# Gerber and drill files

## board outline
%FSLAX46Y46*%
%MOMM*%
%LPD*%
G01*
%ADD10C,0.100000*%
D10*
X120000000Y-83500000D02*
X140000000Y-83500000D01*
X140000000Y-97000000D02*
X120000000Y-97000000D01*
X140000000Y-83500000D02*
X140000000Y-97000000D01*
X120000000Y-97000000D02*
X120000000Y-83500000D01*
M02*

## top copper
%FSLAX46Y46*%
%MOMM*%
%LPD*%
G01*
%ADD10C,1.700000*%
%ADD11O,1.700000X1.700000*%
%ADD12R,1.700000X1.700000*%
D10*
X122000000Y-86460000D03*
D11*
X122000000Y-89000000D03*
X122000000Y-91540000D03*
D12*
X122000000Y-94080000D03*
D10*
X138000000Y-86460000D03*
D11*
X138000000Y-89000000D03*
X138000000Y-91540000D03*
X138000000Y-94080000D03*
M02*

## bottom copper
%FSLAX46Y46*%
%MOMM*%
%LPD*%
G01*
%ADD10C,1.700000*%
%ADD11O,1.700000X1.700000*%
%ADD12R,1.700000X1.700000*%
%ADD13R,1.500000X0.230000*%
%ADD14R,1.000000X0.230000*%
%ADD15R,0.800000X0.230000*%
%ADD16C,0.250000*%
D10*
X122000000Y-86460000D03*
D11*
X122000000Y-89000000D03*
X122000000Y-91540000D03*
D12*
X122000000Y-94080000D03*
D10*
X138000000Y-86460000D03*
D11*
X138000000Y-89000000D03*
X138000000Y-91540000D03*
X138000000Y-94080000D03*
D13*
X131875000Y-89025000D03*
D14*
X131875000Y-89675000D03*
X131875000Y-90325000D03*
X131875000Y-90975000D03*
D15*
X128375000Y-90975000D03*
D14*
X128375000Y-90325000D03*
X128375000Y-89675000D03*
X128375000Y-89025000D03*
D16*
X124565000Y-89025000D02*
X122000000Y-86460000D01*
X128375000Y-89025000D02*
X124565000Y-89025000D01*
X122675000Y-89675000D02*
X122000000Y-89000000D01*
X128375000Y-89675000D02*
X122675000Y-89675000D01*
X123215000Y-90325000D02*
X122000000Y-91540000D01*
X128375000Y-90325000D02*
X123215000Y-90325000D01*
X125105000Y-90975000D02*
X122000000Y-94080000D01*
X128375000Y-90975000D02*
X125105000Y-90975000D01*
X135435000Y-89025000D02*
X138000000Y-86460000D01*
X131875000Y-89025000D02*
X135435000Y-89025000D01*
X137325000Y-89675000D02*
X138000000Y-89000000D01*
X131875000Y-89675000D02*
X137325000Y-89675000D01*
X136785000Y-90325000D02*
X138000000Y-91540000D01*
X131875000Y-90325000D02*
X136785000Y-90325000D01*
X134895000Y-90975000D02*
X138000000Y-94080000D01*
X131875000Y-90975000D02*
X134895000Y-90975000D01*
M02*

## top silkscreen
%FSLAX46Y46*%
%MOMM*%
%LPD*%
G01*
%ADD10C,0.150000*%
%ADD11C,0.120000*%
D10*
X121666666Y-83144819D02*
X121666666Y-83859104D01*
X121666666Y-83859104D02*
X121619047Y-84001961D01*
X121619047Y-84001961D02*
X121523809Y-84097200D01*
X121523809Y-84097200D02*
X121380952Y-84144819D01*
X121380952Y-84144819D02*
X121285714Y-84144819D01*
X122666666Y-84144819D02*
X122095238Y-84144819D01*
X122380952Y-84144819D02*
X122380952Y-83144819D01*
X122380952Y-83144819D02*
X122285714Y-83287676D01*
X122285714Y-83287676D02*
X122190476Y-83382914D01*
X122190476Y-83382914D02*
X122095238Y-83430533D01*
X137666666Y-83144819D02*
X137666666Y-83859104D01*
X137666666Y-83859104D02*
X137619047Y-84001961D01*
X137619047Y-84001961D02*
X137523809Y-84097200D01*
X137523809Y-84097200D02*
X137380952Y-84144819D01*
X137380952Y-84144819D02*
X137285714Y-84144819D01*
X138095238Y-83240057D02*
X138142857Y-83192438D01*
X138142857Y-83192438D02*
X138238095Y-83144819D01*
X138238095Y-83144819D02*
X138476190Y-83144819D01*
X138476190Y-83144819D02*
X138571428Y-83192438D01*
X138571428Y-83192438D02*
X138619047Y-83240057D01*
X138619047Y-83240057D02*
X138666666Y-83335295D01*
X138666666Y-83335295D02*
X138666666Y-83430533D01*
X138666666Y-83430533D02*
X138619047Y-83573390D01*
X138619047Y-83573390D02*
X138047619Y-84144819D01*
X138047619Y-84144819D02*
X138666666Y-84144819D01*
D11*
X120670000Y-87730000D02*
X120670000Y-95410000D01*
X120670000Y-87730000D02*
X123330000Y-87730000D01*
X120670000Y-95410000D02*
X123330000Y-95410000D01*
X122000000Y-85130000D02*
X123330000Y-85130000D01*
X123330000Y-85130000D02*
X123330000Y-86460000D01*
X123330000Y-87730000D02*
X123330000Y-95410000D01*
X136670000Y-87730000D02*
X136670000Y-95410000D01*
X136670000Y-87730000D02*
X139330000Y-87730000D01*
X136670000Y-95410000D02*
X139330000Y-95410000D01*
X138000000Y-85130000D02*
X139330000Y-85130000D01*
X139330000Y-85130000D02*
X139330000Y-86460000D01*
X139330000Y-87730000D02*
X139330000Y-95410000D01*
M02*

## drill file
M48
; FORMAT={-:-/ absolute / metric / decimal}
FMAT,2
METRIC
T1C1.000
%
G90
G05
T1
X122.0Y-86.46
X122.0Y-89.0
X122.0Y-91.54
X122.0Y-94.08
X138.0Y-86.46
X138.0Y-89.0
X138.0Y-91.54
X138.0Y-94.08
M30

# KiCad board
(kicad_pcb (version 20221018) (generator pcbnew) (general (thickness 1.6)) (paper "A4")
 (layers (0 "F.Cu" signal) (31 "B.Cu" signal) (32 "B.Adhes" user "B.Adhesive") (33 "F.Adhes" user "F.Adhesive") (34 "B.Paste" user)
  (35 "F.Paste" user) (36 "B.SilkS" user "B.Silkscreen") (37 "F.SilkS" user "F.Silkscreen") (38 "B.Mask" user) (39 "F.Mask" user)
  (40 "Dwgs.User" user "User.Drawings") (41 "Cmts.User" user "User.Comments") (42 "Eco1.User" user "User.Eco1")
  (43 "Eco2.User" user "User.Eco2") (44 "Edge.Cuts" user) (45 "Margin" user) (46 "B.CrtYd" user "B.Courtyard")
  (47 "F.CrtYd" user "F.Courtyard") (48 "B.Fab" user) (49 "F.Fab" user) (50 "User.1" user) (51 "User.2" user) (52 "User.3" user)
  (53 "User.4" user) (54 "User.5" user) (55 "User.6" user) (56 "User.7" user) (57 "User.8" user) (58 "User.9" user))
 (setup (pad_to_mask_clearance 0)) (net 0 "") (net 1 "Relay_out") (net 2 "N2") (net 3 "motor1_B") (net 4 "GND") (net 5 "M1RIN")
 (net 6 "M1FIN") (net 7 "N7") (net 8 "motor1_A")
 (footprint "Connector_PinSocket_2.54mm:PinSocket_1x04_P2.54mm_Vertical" (layer "F.Cu") (at 122 86.46)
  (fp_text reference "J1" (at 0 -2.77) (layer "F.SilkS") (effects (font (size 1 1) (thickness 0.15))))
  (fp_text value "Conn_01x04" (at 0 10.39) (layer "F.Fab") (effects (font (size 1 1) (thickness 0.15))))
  (fp_line (start -1.33 1.27) (end -1.33 8.95) (stroke (width 0.12) (type solid)) (layer "F.SilkS"))
  (fp_line (start -1.33 1.27) (end 1.33 1.27) (stroke (width 0.12) (type solid)) (layer "F.SilkS"))
  (fp_line (start -1.33 8.95) (end 1.33 8.95) (stroke (width 0.12) (type solid)) (layer "F.SilkS"))
  (fp_line (start 0 -1.33) (end 1.33 -1.33) (stroke (width 0.12) (type solid)) (layer "F.SilkS"))
  (fp_line (start 1.33 -1.33) (end 1.33 0) (stroke (width 0.12) (type solid)) (layer "F.SilkS"))
  (fp_line (start 1.33 1.27) (end 1.33 8.95) (stroke (width 0.12) (type solid)) (layer "F.SilkS"))
  (pad "1" thru_hole circle (at 0 0) (size 1.7 1.7) (drill 1) (layers "*.Cu" "*.Mask") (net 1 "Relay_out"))
  (pad "2" thru_hole oval (at 0 2.54) (size 1.7 1.7) (drill 1) (layers "*.Cu" "*.Mask") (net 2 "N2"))
  (pad "3" thru_hole oval (at 0 5.08) (size 1.7 1.7) (drill 1) (layers "*.Cu" "*.Mask") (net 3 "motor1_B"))
  (pad "4" thru_hole rect (at 0 7.62) (size 1.7 1.7) (drill 1) (layers "*.Cu" "*.Mask") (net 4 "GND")))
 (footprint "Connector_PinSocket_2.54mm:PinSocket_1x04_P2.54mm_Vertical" (layer "F.Cu") (at 138 86.46)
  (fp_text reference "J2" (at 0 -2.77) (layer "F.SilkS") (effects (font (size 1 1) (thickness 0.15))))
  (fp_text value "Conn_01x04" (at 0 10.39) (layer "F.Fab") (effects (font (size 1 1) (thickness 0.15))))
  (fp_line (start -1.33 1.27) (end -1.33 8.95) (stroke (width 0.12) (type solid)) (layer "F.SilkS"))
  (fp_line (start -1.33 1.27) (end 1.33 1.27) (stroke (width 0.12) (type solid)) (layer "F.SilkS"))
  (fp_line (start -1.33 8.95) (end 1.33 8.95) (stroke (width 0.12) (type solid)) (layer "F.SilkS"))
  (fp_line (start 0 -1.33) (end 1.33 -1.33) (stroke (width 0.12) (type solid)) (layer "F.SilkS"))
  (fp_line (start 1.33 -1.33) (end 1.33 0) (stroke (width 0.12) (type solid)) (layer "F.SilkS"))
  (fp_line (start 1.33 1.27) (end 1.33 8.95) (stroke (width 0.12) (type solid)) (layer "F.SilkS"))
  (pad "1" thru_hole circle (at 0 0) (size 1.7 1.7) (drill 1) (layers "*.Cu" "*.Mask") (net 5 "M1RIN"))
  (pad "2" thru_hole oval (at 0 2.54) (size 1.7 1.7) (drill 1) (layers "*.Cu" "*.Mask") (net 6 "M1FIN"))
  (pad "3" thru_hole oval (at 0 5.08) (size 1.7 1.7) (drill 1) (layers "*.Cu" "*.Mask") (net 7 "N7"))
  (pad "4" thru_hole oval (at 0 7.62) (size 1.7 1.7) (drill 1) (layers "*.Cu" "*.Mask") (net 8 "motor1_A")))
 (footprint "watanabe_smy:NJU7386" (layer "B.Cu") (at 127.875 90 -90)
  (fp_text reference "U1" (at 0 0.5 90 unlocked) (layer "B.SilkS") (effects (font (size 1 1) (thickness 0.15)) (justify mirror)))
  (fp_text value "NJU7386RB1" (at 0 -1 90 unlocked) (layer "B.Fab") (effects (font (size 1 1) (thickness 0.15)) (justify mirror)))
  (pad "1" smd rect (at -0.975 -4 270) (size 0.23 1.5) (layers "B.Cu" "B.Paste" "B.Mask") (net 5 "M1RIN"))
  (pad "2" smd rect (at -0.325 -4 270) (size 0.23 1) (layers "B.Cu" "B.Paste" "B.Mask") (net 6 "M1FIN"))
  (pad "3" smd rect (at 0.325 -4 270) (size 0.23 1) (layers "B.Cu" "B.Paste" "B.Mask") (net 7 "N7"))
  (pad "4" smd rect (at 0.975 -4 270) (size 0.23 1) (layers "B.Cu" "B.Paste" "B.Mask") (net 8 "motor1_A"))
  (pad "5" smd rect (at 0.975 -0.5 270) (size 0.23 0.8) (layers "B.Cu" "B.Paste" "B.Mask") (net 4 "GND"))
  (pad "6" smd rect (at 0.325 -0.5 270) (size 0.23 1) (layers "B.Cu" "B.Paste" "B.Mask") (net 3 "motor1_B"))
  (pad "7" smd rect (at -0.325 -0.5 270) (size 0.23 1) (layers "B.Cu" "B.Paste" "B.Mask") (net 2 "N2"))
  (pad "8" smd rect (at -0.975 -0.5 270) (size 0.23 1) (layers "B.Cu" "B.Paste" "B.Mask") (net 1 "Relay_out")))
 (gr_line (start 120 83.5) (end 140 83.5) (stroke (width 0.1) (type default)) (layer "Edge.Cuts"))
 (gr_line (start 140 97) (end 120 97) (stroke (width 0.1) (type default)) (layer "Edge.Cuts"))
 (gr_line (start 140 83.5) (end 140 97) (stroke (width 0.1) (type default)) (layer "Edge.Cuts"))
 (gr_line (start 120 97) (end 120 83.5) (stroke (width 0.1) (type default)) (layer "Edge.Cuts"))
 (segment (start 124.565 89.025) (end 122 86.46) (width 0.25) (layer "B.Cu") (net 1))
 (segment (start 128.375 89.025) (end 124.565 89.025) (width 0.25) (layer "B.Cu") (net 1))
 (segment (start 122.675 89.675) (end 122 89) (width 0.25) (layer "B.Cu") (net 2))
 (segment (start 128.375 89.675) (end 122.675 89.675) (width 0.25) (layer "B.Cu") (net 2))
 (segment (start 123.215 90.325) (end 122 91.54) (width 0.25) (layer "B.Cu") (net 3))
 (segment (start 128.375 90.325) (end 123.215 90.325) (width 0.25) (layer "B.Cu") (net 3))
 (segment (start 125.105 90.975) (end 122 94.08) (width 0.25) (layer "B.Cu") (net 4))
 (segment (start 128.375 90.975) (end 125.105 90.975) (width 0.25) (layer "B.Cu") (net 4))
 (segment (start 135.435 89.025) (end 138 86.46) (width 0.25) (layer "B.Cu") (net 5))
 (segment (start 131.875 89.025) (end 135.435 89.025) (width 0.25) (layer "B.Cu") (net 5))
 (segment (start 137.325 89.675) (end 138 89) (width 0.25) (layer "B.Cu") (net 6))
 (segment (start 131.875 89.675) (end 137.325 89.675) (width 0.25) (layer "B.Cu") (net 6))
 (segment (start 136.785 90.325) (end 138 91.54) (width 0.25) (layer "B.Cu") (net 7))
 (segment (start 131.875 90.325) (end 136.785 90.325) (width 0.25) (layer "B.Cu") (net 7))
 (segment (start 134.895 90.975) (end 138 94.08) (width 0.25) (layer "B.Cu") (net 8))
 (segment (start 131.875 90.975) (end 134.895 90.975) (width 0.25) (layer "B.Cu") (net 8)))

